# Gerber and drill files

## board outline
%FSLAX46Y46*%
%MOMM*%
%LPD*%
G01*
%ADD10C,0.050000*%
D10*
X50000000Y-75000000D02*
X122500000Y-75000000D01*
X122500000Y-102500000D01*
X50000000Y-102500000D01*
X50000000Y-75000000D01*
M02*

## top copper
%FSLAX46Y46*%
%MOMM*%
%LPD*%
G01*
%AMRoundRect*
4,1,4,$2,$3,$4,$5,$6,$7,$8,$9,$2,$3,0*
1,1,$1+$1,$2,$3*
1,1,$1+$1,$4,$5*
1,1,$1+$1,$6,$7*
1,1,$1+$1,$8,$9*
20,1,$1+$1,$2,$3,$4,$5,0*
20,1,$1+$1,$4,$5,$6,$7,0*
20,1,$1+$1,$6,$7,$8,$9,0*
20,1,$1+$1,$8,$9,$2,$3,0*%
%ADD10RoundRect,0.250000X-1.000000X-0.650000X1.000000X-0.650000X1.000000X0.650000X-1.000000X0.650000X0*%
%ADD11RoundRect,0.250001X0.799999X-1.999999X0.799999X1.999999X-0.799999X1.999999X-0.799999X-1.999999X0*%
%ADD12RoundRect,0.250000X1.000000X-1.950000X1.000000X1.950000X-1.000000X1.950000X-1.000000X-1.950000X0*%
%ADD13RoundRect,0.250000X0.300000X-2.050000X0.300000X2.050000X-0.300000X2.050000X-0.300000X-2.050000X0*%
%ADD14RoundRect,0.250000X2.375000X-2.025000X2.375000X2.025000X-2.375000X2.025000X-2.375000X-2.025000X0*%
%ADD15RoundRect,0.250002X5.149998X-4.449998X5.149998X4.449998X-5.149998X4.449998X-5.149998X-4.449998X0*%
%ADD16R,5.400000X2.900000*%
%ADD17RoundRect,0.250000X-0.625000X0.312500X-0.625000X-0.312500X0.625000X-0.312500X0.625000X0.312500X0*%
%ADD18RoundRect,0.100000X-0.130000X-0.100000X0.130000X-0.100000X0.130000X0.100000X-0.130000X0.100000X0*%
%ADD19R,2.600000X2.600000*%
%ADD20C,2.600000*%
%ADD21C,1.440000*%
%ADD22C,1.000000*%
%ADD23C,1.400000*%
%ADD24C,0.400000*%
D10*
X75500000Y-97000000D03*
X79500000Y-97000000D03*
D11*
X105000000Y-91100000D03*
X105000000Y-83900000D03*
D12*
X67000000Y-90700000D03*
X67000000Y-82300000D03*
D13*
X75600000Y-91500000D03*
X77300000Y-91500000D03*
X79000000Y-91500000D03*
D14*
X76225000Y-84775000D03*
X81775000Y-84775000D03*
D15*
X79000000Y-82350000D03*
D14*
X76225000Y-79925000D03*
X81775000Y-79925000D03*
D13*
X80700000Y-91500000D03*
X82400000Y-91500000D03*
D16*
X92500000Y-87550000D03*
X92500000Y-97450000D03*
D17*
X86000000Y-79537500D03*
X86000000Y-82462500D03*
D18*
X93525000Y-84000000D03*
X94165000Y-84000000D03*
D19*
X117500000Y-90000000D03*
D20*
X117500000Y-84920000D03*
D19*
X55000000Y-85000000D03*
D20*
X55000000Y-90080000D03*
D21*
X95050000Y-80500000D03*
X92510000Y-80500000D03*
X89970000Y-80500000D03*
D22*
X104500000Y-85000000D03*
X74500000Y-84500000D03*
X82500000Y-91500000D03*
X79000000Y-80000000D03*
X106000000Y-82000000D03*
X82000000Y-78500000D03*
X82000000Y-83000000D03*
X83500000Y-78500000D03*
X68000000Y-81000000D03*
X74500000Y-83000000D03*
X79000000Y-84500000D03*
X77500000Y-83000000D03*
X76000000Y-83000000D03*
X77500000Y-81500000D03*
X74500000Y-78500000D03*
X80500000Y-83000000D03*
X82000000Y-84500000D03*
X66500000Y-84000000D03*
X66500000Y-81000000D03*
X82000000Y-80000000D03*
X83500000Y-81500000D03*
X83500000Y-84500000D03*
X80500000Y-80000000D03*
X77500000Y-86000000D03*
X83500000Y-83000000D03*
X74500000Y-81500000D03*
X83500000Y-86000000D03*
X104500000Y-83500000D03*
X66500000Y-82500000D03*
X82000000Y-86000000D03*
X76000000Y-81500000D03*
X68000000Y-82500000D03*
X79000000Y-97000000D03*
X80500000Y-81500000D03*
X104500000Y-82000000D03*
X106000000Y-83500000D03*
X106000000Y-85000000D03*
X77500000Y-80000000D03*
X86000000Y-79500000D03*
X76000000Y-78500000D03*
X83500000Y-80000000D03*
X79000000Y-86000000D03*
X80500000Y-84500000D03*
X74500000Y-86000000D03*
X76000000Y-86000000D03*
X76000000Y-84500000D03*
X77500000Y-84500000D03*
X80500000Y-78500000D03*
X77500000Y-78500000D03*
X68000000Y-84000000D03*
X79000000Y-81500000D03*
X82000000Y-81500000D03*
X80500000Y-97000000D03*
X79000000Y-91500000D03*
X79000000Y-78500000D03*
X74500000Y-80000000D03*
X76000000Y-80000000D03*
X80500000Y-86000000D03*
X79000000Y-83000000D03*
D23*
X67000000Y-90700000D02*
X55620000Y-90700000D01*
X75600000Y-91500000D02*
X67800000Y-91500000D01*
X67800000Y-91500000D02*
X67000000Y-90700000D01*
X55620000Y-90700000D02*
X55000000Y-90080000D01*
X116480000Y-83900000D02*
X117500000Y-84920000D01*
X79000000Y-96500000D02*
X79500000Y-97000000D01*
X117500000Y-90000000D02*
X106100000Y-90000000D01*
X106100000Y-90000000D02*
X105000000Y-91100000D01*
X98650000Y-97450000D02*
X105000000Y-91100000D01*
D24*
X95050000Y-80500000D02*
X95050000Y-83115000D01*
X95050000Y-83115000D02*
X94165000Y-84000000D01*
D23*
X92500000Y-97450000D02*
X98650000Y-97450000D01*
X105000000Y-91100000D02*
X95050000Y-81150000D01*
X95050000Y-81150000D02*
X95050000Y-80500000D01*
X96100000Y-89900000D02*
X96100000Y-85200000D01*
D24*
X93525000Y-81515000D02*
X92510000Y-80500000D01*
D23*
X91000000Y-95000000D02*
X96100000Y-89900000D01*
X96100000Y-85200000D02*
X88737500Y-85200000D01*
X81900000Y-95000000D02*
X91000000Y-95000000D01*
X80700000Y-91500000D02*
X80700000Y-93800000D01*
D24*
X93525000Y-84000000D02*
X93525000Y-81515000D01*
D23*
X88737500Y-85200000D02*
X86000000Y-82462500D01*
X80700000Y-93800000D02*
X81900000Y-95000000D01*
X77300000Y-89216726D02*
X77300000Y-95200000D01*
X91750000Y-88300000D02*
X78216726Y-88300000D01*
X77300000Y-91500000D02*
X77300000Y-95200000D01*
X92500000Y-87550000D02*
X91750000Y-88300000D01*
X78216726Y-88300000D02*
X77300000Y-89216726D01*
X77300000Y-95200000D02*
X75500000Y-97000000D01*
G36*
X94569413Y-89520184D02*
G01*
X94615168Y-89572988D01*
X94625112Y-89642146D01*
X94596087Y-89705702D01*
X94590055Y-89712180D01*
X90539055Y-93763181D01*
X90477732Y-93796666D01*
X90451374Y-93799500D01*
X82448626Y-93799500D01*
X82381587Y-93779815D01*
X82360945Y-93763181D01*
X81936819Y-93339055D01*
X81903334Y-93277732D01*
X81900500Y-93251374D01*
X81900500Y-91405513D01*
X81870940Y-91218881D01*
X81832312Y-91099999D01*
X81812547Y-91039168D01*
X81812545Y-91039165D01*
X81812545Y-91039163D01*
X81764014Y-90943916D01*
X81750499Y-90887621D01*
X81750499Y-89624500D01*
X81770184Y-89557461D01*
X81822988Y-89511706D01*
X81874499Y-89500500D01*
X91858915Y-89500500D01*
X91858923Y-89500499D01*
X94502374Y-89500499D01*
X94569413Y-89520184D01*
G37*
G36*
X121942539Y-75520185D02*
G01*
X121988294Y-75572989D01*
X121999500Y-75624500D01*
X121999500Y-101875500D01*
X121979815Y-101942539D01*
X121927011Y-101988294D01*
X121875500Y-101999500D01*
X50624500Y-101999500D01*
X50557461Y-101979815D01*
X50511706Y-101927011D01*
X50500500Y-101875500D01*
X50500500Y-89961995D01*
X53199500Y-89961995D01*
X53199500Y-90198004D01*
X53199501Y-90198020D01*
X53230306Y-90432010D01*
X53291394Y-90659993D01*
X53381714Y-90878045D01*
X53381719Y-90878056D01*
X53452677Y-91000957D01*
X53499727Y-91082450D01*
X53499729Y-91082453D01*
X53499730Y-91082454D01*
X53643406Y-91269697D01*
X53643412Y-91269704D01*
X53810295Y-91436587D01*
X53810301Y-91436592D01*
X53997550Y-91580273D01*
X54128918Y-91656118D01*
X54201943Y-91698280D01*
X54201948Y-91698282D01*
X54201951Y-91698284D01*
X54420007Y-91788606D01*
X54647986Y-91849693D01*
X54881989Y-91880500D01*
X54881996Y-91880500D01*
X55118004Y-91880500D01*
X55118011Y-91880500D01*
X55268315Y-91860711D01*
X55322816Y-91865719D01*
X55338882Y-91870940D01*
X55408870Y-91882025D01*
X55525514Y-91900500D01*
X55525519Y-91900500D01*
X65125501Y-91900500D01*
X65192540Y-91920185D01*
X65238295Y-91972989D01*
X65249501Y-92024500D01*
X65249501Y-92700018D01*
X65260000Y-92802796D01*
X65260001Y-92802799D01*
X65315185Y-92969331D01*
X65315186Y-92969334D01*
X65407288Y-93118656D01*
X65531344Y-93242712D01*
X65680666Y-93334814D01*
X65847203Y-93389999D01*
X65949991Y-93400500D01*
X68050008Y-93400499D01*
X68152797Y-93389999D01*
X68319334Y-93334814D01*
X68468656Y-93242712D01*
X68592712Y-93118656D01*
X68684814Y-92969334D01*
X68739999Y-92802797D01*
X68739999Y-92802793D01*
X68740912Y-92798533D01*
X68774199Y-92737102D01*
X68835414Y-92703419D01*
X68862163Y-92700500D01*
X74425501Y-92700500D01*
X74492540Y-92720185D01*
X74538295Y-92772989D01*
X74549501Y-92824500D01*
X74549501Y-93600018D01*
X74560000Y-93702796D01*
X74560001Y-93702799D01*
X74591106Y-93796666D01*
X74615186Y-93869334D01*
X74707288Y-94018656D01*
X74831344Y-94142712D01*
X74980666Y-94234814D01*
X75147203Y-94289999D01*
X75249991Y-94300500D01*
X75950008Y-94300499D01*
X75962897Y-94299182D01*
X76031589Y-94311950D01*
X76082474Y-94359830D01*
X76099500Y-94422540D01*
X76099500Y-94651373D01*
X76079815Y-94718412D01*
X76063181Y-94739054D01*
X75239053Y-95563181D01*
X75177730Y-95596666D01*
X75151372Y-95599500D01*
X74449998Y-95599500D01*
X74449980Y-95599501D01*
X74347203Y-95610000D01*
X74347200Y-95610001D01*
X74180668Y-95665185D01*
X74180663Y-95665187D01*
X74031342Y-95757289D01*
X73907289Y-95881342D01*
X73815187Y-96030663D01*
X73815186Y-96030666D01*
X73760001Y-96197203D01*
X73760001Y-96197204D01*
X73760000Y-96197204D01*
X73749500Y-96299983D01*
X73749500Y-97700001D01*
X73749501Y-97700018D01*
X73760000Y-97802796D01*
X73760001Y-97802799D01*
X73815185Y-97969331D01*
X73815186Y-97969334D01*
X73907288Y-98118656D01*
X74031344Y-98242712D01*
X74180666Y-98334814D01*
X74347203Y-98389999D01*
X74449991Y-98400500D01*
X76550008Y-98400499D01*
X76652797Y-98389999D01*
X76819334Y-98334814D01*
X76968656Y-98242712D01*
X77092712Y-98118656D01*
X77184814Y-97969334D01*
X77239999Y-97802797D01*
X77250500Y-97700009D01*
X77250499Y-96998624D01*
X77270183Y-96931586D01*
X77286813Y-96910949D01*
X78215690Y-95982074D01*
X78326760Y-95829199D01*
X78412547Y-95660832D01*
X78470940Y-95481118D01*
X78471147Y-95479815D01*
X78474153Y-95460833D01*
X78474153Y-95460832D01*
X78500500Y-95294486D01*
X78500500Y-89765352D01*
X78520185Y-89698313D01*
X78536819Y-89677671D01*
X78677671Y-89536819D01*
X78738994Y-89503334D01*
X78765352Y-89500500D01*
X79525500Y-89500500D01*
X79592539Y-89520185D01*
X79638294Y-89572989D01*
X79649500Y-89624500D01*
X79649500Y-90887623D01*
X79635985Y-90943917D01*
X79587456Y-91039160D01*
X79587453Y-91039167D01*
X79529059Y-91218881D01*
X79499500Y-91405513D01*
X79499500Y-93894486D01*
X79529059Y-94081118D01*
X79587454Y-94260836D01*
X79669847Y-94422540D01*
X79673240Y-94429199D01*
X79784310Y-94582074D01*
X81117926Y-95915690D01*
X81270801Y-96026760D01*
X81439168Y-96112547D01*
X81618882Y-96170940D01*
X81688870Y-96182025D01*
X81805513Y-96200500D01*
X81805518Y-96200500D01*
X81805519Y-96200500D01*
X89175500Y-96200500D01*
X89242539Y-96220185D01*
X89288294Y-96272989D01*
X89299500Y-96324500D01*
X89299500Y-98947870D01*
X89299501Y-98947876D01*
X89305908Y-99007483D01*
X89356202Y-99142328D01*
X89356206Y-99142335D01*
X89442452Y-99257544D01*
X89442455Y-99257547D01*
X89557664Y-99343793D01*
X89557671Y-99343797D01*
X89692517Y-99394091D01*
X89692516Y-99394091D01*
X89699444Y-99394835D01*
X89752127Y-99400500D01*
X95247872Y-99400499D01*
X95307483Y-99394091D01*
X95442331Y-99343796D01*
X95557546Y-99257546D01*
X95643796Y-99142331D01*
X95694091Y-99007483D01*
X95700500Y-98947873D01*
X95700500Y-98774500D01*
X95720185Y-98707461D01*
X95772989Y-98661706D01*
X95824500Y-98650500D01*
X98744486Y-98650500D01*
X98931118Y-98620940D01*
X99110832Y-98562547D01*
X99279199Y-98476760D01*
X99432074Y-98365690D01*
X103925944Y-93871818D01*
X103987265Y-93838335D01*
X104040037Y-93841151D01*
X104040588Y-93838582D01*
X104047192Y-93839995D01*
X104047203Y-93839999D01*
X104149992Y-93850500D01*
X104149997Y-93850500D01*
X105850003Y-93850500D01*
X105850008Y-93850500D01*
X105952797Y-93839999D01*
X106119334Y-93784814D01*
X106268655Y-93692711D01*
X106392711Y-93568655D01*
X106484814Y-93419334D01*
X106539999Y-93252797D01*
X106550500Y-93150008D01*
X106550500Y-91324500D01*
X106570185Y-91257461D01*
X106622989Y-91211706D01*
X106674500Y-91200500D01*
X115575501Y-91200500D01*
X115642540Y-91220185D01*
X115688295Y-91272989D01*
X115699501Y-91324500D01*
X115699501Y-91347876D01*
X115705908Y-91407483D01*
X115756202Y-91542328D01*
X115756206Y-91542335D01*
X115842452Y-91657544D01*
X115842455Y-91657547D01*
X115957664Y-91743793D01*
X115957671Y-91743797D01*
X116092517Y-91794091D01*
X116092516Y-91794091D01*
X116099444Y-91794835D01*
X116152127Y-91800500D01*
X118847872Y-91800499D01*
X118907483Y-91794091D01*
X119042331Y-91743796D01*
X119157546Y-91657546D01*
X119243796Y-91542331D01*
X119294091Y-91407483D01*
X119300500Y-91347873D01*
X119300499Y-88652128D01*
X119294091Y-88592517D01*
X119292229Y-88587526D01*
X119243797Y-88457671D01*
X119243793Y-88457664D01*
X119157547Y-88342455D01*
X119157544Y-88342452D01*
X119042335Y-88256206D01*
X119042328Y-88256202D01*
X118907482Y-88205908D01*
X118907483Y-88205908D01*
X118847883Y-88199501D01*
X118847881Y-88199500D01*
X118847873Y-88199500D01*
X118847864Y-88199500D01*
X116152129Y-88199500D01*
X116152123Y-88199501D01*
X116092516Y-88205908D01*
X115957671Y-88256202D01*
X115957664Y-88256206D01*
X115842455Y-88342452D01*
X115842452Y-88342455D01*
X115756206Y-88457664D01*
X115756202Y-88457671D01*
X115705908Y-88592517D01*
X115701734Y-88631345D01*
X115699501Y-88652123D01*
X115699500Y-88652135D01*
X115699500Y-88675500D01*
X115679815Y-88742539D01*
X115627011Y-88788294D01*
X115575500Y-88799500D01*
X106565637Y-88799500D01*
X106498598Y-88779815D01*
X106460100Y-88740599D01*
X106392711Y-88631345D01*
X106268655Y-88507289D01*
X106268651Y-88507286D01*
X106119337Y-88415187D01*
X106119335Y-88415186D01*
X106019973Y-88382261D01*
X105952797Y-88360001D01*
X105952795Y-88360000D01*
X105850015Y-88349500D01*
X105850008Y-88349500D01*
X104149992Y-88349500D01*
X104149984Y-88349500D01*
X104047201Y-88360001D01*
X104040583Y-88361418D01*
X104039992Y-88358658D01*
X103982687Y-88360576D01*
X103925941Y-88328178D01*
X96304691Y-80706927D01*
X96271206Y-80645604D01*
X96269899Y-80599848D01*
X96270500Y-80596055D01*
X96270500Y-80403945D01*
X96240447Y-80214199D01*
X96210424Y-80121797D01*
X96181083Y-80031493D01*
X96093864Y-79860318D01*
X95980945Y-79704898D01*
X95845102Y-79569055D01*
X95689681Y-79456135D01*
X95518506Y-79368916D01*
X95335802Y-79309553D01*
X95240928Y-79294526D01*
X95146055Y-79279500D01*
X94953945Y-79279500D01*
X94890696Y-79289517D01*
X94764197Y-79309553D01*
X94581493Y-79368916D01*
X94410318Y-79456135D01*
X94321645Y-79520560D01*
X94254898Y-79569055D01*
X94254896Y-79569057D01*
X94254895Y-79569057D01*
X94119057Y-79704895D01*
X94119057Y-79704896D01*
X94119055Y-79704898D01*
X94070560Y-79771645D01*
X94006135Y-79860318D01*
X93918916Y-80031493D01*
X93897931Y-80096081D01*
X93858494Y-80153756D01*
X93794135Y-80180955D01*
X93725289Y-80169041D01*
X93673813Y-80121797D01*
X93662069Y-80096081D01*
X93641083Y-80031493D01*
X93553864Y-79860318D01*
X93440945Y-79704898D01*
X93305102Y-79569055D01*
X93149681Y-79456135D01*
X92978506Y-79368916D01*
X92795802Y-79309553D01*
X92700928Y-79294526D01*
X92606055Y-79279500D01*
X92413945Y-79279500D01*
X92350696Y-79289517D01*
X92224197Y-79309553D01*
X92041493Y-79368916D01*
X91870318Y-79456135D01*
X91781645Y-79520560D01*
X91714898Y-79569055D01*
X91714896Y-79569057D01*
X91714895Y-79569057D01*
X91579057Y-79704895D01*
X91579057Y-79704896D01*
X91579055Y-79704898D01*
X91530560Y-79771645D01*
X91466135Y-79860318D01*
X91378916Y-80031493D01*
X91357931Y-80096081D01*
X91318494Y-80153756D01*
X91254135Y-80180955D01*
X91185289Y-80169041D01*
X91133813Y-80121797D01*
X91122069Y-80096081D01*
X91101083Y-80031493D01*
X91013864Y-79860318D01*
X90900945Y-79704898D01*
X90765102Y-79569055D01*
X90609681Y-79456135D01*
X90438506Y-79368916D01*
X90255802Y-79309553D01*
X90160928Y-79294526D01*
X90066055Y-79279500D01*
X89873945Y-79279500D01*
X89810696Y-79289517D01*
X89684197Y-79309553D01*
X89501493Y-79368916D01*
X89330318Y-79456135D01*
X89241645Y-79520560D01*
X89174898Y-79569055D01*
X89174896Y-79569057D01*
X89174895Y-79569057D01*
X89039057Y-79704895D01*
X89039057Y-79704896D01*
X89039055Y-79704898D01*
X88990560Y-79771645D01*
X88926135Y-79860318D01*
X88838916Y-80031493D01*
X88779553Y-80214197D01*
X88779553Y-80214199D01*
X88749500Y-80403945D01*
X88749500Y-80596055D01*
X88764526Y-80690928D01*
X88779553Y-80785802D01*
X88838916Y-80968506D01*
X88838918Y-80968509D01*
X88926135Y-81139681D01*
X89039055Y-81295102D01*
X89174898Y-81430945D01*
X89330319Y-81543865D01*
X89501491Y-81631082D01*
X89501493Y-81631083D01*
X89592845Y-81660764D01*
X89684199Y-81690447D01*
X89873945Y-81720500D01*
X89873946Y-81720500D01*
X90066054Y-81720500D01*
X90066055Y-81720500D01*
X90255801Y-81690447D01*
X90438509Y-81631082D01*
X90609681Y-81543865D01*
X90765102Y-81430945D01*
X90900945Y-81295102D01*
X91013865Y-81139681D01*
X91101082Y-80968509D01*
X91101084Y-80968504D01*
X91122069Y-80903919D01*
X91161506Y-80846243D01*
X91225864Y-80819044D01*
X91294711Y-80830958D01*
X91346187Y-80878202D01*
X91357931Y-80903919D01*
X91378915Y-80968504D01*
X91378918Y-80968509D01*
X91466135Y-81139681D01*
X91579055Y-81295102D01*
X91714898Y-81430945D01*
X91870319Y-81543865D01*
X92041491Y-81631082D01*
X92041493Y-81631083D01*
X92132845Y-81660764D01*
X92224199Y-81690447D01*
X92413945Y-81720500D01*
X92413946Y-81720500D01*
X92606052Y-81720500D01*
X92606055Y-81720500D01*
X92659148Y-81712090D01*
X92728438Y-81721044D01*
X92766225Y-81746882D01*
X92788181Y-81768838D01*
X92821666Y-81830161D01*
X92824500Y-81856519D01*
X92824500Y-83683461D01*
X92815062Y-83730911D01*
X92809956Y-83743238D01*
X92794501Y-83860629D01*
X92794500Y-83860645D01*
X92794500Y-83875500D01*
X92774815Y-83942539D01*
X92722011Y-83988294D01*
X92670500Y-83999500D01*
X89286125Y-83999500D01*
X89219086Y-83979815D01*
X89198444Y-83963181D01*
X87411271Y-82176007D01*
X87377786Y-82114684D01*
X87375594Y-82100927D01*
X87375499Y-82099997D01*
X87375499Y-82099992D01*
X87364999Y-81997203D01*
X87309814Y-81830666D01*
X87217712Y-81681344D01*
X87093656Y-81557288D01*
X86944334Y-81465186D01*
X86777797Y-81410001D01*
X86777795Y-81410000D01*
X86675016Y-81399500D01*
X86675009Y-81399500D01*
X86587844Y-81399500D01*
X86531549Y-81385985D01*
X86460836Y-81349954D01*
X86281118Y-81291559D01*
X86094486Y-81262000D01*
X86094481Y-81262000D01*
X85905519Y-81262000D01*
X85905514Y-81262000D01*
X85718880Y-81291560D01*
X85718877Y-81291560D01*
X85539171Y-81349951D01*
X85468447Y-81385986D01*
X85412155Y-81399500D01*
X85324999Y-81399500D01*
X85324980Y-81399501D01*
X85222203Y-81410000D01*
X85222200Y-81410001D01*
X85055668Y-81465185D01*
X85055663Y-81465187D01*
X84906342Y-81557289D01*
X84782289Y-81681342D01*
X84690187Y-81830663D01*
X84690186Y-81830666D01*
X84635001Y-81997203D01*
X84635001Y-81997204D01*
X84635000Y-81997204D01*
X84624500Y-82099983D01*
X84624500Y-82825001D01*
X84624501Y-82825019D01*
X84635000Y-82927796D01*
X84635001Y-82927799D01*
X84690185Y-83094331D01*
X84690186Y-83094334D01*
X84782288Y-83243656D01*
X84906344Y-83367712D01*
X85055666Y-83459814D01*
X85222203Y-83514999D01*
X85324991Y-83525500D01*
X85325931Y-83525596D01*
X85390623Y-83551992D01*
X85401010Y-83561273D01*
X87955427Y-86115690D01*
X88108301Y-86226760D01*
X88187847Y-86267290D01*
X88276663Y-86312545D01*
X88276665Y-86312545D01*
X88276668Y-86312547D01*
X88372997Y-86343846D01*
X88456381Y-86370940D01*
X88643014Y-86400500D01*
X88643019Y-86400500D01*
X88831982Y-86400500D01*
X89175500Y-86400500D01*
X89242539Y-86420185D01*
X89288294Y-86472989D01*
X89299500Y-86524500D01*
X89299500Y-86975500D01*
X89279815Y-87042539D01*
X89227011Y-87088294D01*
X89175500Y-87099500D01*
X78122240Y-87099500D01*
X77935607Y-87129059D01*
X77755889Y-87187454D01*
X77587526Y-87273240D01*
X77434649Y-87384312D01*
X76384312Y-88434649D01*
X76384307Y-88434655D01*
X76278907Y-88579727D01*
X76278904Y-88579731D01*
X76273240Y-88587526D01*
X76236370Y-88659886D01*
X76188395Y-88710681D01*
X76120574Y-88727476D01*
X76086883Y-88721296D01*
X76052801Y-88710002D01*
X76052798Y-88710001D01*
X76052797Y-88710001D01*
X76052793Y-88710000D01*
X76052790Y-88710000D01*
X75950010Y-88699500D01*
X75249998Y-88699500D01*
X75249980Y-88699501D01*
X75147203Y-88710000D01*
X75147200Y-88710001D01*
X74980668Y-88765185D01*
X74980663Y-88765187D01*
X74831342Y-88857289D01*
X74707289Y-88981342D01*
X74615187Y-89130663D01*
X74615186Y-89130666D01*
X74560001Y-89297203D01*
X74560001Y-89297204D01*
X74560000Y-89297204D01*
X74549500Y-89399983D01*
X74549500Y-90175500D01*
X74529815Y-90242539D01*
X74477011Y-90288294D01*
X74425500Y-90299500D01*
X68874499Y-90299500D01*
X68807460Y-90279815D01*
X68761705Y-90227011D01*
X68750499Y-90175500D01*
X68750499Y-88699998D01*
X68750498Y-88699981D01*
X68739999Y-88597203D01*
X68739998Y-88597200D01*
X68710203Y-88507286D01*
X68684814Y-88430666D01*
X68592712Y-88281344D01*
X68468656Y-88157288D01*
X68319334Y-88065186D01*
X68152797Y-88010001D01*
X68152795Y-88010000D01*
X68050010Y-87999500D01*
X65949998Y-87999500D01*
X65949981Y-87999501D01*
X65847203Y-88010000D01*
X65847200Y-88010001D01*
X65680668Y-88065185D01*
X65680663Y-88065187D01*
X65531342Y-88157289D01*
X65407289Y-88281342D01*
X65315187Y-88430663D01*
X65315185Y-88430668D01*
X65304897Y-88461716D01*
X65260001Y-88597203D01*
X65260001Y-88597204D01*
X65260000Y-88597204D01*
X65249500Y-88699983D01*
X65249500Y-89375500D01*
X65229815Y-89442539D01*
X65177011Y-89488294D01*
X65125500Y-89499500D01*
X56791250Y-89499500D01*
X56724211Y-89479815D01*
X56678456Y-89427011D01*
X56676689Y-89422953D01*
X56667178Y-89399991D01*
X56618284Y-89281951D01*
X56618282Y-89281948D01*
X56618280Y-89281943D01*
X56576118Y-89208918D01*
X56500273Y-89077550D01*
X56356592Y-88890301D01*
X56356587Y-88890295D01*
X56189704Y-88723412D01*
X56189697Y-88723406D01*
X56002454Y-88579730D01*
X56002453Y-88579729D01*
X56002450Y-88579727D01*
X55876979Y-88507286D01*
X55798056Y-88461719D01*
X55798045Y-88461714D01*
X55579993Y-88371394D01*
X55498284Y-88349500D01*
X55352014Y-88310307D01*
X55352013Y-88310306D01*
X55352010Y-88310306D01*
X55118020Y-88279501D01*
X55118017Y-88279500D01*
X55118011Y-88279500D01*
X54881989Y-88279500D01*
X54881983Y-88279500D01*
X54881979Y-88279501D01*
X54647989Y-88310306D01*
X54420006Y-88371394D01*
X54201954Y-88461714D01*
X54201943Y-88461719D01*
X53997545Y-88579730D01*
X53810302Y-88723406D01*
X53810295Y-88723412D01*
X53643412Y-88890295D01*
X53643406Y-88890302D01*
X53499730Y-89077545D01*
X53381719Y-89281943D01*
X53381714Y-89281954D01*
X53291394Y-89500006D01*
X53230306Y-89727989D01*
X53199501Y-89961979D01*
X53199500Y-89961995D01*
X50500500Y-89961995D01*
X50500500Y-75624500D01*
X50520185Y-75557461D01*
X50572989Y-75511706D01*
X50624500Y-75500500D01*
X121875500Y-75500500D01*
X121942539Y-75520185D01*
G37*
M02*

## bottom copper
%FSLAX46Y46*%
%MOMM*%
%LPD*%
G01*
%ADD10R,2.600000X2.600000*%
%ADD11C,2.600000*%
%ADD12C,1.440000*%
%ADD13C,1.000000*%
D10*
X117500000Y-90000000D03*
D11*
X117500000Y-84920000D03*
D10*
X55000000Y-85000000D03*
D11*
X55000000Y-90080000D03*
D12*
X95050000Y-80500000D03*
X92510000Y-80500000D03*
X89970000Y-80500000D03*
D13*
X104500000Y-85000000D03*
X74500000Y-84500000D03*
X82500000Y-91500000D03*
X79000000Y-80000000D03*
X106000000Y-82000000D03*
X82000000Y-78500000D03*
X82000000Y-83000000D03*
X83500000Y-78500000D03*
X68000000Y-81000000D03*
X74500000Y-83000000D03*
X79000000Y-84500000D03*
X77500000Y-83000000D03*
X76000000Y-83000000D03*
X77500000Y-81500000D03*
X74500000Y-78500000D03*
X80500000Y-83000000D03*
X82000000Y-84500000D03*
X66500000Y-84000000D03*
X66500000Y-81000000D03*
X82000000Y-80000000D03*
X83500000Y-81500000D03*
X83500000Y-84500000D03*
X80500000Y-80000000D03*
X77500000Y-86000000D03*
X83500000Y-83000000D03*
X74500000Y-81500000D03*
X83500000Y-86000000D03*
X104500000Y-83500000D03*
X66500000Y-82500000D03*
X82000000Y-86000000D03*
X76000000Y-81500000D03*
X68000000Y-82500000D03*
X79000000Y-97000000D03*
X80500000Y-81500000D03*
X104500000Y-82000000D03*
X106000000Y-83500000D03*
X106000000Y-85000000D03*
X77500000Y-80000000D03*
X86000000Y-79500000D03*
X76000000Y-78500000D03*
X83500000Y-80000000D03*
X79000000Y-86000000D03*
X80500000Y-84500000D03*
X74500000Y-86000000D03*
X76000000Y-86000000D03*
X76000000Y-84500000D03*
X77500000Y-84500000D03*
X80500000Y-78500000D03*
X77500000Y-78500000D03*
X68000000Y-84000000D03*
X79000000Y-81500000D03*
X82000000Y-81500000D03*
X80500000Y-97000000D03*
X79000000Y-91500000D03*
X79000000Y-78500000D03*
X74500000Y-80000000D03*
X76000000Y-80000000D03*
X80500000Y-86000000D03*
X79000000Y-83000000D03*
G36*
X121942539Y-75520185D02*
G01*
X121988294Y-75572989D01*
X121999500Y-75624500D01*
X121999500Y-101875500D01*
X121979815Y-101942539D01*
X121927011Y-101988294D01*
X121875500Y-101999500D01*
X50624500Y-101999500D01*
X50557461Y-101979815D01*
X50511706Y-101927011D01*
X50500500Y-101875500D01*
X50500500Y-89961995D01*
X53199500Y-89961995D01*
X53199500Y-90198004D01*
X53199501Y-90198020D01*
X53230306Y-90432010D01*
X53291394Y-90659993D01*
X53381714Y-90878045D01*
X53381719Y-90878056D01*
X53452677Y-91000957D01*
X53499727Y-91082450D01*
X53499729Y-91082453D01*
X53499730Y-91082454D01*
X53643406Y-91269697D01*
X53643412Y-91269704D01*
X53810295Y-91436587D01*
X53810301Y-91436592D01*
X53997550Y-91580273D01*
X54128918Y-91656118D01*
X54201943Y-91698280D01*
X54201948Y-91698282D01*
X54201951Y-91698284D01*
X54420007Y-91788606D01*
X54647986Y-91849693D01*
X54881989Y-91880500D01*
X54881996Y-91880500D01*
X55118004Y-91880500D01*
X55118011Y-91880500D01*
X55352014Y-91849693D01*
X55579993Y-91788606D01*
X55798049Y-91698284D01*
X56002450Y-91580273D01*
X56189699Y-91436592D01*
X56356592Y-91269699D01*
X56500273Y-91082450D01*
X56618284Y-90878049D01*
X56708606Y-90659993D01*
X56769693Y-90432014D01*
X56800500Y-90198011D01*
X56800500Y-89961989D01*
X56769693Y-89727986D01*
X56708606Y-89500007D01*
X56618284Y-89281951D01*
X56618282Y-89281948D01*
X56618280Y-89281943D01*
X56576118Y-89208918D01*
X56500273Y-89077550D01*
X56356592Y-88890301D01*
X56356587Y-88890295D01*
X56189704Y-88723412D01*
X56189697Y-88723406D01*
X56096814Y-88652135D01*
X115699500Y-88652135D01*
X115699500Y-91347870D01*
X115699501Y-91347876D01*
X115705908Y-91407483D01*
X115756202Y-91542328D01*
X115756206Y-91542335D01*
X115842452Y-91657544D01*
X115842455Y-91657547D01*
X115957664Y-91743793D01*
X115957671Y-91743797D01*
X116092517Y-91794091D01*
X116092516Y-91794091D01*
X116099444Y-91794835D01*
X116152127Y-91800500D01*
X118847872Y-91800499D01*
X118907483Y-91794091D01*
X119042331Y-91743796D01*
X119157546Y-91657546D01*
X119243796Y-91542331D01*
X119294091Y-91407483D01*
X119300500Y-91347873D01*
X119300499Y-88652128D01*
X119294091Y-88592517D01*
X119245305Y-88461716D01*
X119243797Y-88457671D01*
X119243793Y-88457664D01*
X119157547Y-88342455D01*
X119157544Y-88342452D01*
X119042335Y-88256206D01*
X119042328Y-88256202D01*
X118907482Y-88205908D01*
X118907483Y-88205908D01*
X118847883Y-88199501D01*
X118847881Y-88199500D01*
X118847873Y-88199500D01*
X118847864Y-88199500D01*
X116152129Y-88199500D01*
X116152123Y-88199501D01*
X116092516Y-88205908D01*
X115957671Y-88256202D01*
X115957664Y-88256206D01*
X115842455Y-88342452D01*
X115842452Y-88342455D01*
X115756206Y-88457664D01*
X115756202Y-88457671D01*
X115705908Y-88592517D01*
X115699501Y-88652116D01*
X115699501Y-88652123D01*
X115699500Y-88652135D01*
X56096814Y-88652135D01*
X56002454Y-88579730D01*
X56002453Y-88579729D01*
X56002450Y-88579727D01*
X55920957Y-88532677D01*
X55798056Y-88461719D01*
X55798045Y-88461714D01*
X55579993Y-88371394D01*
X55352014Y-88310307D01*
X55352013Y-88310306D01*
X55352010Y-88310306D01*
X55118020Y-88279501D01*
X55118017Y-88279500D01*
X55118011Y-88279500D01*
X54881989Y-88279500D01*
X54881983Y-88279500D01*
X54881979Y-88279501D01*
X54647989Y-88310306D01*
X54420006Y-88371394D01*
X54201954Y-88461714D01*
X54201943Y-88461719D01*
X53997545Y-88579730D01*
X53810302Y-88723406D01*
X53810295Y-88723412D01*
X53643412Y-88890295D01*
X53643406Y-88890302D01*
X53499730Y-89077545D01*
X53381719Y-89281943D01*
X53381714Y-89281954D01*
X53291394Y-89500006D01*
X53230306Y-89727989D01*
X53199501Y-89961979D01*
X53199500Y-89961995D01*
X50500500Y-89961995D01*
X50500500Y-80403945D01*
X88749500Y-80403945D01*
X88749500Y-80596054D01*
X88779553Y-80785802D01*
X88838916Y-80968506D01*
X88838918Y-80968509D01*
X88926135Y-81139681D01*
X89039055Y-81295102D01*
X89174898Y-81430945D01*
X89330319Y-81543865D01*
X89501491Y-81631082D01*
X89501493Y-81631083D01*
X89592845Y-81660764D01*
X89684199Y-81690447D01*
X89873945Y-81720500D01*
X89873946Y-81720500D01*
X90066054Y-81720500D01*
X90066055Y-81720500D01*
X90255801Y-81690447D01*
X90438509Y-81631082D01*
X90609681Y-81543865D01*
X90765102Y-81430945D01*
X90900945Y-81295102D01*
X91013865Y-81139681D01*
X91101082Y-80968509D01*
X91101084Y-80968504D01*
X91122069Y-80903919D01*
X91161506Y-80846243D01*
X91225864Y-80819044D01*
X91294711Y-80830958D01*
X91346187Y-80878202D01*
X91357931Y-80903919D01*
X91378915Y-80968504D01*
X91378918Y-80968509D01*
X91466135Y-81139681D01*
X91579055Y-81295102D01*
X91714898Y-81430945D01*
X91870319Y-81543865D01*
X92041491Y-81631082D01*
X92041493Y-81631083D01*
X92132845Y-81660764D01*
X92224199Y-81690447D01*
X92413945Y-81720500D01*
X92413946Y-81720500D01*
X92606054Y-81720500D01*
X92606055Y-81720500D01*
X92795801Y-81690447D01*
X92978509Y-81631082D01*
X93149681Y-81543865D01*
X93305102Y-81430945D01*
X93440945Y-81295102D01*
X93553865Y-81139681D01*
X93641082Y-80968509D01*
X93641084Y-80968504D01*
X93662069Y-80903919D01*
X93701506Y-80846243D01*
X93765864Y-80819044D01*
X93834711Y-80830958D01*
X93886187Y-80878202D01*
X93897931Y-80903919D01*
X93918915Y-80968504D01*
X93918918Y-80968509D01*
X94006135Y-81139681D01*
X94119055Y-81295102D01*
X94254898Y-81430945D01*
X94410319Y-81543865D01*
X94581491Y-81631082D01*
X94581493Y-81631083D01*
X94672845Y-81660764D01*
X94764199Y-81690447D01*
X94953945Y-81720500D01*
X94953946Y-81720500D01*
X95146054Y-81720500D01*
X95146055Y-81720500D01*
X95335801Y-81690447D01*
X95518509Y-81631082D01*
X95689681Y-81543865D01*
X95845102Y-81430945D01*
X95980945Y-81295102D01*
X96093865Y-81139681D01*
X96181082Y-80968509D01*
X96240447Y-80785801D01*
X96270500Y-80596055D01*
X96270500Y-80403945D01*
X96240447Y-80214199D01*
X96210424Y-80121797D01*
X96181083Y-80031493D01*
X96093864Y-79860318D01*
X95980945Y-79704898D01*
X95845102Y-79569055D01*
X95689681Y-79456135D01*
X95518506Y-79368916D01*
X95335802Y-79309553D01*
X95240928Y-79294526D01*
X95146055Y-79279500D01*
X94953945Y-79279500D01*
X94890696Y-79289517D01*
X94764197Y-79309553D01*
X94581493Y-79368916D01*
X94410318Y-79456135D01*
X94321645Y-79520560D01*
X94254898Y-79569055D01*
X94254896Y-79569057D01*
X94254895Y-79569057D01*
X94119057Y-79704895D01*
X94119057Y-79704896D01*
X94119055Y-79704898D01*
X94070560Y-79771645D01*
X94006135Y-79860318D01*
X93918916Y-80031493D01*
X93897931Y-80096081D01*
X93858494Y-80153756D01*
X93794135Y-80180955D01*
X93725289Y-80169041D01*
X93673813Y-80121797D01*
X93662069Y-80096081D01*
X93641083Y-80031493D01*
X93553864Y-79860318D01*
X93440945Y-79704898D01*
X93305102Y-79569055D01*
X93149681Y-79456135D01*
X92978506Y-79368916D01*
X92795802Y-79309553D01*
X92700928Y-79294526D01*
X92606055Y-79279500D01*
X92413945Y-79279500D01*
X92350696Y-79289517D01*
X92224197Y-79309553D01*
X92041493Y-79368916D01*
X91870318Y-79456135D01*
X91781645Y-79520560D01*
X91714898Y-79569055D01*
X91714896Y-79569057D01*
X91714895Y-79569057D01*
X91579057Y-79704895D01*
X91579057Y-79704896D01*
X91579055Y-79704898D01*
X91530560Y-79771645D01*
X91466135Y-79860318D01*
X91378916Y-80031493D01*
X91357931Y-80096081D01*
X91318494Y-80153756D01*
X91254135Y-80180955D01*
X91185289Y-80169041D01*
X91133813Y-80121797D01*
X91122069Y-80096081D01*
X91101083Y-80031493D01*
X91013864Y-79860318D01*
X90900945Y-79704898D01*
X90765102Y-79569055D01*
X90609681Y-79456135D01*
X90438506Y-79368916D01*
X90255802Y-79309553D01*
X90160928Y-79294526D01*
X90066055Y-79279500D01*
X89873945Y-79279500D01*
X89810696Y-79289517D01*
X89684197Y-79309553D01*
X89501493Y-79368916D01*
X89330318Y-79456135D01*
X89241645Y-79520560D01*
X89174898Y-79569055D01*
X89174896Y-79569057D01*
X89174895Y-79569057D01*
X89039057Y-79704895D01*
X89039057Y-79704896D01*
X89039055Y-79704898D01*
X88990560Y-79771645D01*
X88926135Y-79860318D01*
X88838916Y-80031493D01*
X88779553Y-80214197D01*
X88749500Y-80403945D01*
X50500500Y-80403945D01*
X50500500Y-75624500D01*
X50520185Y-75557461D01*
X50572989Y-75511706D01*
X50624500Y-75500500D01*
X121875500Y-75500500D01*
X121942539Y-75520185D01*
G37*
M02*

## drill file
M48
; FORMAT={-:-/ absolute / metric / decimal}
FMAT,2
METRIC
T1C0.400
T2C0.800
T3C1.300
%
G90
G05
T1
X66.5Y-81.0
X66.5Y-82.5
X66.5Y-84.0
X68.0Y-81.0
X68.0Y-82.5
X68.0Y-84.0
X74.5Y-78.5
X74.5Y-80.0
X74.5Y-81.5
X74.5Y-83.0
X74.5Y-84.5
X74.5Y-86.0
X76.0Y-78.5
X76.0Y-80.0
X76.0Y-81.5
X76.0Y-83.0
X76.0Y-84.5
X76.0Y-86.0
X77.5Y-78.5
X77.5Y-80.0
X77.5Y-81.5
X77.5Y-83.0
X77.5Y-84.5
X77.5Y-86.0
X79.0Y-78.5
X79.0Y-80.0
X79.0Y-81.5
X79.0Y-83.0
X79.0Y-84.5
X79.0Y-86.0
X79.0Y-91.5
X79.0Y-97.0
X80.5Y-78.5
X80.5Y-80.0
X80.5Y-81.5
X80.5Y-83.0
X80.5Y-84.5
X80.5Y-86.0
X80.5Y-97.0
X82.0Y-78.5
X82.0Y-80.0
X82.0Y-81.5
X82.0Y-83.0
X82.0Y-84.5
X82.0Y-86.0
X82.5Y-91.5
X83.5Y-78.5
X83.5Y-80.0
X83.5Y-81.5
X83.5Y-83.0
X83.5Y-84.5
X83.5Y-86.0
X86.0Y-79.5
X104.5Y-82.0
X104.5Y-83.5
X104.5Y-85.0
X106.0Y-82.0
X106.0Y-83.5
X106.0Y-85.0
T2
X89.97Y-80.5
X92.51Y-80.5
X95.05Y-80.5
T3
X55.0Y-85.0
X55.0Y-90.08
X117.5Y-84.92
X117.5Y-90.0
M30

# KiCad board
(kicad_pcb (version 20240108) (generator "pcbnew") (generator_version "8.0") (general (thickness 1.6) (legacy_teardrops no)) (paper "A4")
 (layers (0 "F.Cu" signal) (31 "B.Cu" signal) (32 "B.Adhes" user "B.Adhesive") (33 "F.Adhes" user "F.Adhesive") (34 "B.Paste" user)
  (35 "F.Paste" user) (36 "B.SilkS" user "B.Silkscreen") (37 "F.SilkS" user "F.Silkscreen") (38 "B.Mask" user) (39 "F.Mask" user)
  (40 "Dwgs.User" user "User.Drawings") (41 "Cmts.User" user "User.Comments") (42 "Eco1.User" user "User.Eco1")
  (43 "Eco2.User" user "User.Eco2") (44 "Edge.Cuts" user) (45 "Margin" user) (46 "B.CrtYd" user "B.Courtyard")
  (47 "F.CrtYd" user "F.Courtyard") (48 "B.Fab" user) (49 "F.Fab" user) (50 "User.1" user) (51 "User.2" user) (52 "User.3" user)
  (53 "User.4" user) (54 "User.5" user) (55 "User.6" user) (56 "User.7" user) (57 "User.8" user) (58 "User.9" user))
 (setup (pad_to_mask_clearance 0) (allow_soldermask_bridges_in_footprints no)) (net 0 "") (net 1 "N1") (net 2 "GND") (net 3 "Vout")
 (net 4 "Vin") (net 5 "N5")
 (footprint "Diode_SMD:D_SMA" (layer "F.Cu") (at 77.5 97)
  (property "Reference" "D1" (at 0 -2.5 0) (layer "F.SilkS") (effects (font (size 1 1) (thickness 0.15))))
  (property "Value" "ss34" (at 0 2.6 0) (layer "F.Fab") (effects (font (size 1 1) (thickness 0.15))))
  (pad "1" smd roundrect (at -2 0) (size 2.5 1.8) (layers "F.Cu" "F.Paste" "F.Mask") (roundrect_rratio 0.1388888889) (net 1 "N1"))
  (pad "2" smd roundrect (at 2 0) (size 2.5 1.8) (layers "F.Cu" "F.Paste" "F.Mask") (roundrect_rratio 0.1388888889) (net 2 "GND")))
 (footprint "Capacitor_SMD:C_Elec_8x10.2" (layer "F.Cu") (at 105 87.5 90)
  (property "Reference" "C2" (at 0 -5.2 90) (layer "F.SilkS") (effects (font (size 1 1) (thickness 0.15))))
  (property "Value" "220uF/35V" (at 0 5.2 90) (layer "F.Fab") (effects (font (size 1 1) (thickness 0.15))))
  (pad "1" smd roundrect (at -3.6 0 90) (size 4.5 2.1) (layers "F.Cu" "F.Paste" "F.Mask") (roundrect_rratio 0.119048) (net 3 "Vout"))
  (pad "2" smd roundrect (at 3.6 0 90) (size 4.5 2.1) (layers "F.Cu" "F.Paste" "F.Mask") (roundrect_rratio 0.119048) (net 2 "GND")))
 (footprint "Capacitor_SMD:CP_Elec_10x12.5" (layer "F.Cu") (at 67 86.5 90)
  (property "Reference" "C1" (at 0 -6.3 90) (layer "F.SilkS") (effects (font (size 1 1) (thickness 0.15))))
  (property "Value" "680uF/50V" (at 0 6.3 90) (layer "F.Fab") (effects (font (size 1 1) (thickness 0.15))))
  (pad "1" smd roundrect (at -4.2 0 90) (size 4.4 2.5) (layers "F.Cu" "F.Paste" "F.Mask") (roundrect_rratio 0.1) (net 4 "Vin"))
  (pad "2" smd roundrect (at 4.2 0 90) (size 4.4 2.5) (layers "F.Cu" "F.Paste" "F.Mask") (roundrect_rratio 0.1) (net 2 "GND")))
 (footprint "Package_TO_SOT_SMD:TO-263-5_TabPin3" (layer "F.Cu") (at 79 83.85 90)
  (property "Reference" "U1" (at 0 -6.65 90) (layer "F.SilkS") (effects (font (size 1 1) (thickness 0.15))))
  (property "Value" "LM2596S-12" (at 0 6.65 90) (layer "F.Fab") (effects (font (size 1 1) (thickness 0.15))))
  (pad "1" smd roundrect (at -7.65 -3.4 90) (size 4.6 1.1) (layers "F.Cu" "F.Paste" "F.Mask") (roundrect_rratio 0.227273) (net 4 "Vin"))
  (pad "2" smd roundrect (at -7.65 -1.7 90) (size 4.6 1.1) (layers "F.Cu" "F.Paste" "F.Mask") (roundrect_rratio 0.227273) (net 1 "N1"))
  (pad "3" smd roundrect (at -7.65 0 90) (size 4.6 1.1) (layers "F.Cu" "F.Paste" "F.Mask") (roundrect_rratio 0.227273) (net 2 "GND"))
  (pad "3" smd roundrect (at -0.925 -2.775 90) (size 4.55 5.25) (layers "F.Cu" "F.Paste") (roundrect_rratio 0.054945) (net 2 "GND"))
  (pad "3" smd roundrect (at -0.925 2.775 90) (size 4.55 5.25) (layers "F.Cu" "F.Paste") (roundrect_rratio 0.054945) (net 2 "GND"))
  (pad "3" smd roundrect (at 1.5 0 90) (size 9.4 10.8) (layers "F.Cu" "F.Mask") (roundrect_rratio 0.026596) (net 2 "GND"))
  (pad "3" smd roundrect (at 3.925 -2.775 90) (size 4.55 5.25) (layers "F.Cu" "F.Paste") (roundrect_rratio 0.054945) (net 2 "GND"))
  (pad "3" smd roundrect (at 3.925 2.775 90) (size 4.55 5.25) (layers "F.Cu" "F.Paste") (roundrect_rratio 0.054945) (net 2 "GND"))
  (pad "4" smd roundrect (at -7.65 1.7 90) (size 4.6 1.1) (layers "F.Cu" "F.Paste" "F.Mask") (roundrect_rratio 0.227273) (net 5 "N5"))
  (pad "5" smd roundrect (at -7.65 3.4 90) (size 4.6 1.1) (layers "F.Cu" "F.Paste" "F.Mask") (roundrect_rratio 0.227273) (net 2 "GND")))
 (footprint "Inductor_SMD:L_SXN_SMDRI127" (layer "F.Cu") (at 92.5 92.5 -90)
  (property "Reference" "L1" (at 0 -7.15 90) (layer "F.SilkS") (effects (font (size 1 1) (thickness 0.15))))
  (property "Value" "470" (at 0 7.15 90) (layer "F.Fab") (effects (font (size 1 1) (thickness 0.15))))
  (pad "1" smd rect (at -4.95 0 270) (size 2.9 5.4) (layers "F.Cu" "F.Paste" "F.Mask") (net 1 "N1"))
  (pad "2" smd rect (at 4.95 0 270) (size 2.9 5.4) (layers "F.Cu" "F.Paste" "F.Mask") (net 3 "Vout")))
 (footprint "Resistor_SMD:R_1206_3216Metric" (layer "F.Cu") (at 86 81 -90)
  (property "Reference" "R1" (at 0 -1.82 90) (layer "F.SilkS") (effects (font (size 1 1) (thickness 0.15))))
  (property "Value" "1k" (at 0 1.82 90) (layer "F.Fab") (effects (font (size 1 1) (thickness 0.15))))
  (pad "1" smd roundrect (at -1.4625 0 270) (size 1.125 1.75) (layers "F.Cu" "F.Paste" "F.Mask") (roundrect_rratio 0.222222) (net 2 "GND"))
  (pad "2" smd roundrect (at 1.4625 0 270) (size 1.125 1.75) (layers "F.Cu" "F.Paste" "F.Mask") (roundrect_rratio 0.222222) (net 5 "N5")))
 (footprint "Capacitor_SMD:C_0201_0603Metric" (layer "F.Cu") (at 93.845 84)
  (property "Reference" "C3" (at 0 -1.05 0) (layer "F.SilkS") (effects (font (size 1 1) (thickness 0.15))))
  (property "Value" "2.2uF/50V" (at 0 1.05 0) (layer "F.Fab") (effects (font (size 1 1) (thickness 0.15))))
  (pad "" smd roundrect (at -0.345 0) (size 0.318 0.36) (layers "F.Paste") (roundrect_rratio 0.25))
  (pad "" smd roundrect (at 0.345 0) (size 0.318 0.36) (layers "F.Paste") (roundrect_rratio 0.25))
  (pad "1" smd roundrect (at -0.32 0) (size 0.46 0.4) (layers "F.Cu" "F.Mask") (roundrect_rratio 0.25) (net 5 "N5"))
  (pad "2" smd roundrect (at 0.32 0) (size 0.46 0.4) (layers "F.Cu" "F.Mask") (roundrect_rratio 0.25) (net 3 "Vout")))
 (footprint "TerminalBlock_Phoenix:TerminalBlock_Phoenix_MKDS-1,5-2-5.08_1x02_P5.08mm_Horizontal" (layer "F.Cu") (at 117.5 90 90)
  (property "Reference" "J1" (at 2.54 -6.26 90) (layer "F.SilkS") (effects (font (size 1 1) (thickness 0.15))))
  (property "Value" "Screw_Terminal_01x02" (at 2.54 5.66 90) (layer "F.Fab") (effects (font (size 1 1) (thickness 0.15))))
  (pad "1" thru_hole rect (at 0 0 90) (size 2.6 2.6) (drill 1.3) (layers "*.Cu" "*.Mask") (remove_unused_layers no) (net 3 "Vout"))
  (pad "2" thru_hole circle (at 5.08 0 90) (size 2.6 2.6) (drill 1.3) (layers "*.Cu" "*.Mask") (remove_unused_layers no) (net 2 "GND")))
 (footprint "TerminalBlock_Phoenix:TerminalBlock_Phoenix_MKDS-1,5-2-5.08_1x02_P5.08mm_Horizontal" (layer "F.Cu") (at 55 85 -90)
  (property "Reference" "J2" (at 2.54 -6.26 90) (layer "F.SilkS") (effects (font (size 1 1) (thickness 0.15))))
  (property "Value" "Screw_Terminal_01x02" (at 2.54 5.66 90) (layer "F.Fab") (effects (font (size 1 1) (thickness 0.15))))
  (pad "1" thru_hole rect (at 0 0 270) (size 2.6 2.6) (drill 1.3) (layers "*.Cu" "*.Mask") (remove_unused_layers no) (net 2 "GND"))
  (pad "2" thru_hole circle (at 5.08 0 270) (size 2.6 2.6) (drill 1.3) (layers "*.Cu" "*.Mask") (remove_unused_layers no) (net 4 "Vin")))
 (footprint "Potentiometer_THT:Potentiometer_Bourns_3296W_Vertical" (layer "F.Cu") (at 95.05 80.5)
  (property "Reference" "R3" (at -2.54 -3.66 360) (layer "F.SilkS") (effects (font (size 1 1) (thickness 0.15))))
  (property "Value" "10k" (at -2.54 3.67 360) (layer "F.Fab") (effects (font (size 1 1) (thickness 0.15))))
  (pad "1" thru_hole circle (at 0 0) (size 1.44 1.44) (drill 0.8) (layers "*.Cu" "*.Mask") (remove_unused_layers no) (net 3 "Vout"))
  (pad "2" thru_hole circle (at -2.54 0) (size 1.44 1.44) (drill 0.8) (layers "*.Cu" "*.Mask") (remove_unused_layers no) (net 5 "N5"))
  (pad "3" thru_hole circle (at -5.08 0) (size 1.44 1.44) (drill 0.8) (layers "*.Cu" "*.Mask") (remove_unused_layers no)))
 (gr_rect (start 50 75) (end 122.5 102.5) (stroke (width 0.05) (type default)) (fill none) (layer "Edge.Cuts"))
 (segment (start 67 90.7) (end 55.62 90.7) (width 1.4) (layer "F.Cu") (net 4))
 (segment (start 75.6 91.5) (end 67.8 91.5) (width 1.4) (layer "F.Cu") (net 4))
 (segment (start 67.8 91.5) (end 67 90.7) (width 1.4) (layer "F.Cu") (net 4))
 (segment (start 55.62 90.7) (end 55 90.08) (width 1.4) (layer "F.Cu") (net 4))
 (segment (start 116.48 83.9) (end 117.5 84.92) (width 1.4) (layer "F.Cu") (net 2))
 (segment (start 79 96.5) (end 79.5 97) (width 1.4) (layer "F.Cu") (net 2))
 (via (at 104.5 85) (size 1) (drill 0.4) (layers "F.Cu" "B.Cu") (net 2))
 (via (at 74.5 84.5) (size 1) (drill 0.4) (layers "F.Cu" "B.Cu") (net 2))
 (via (at 82.5 91.5) (size 1) (drill 0.4) (layers "F.Cu" "B.Cu") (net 2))
 (via (at 79 80) (size 1) (drill 0.4) (layers "F.Cu" "B.Cu") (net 2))
 (via (at 106 82) (size 1) (drill 0.4) (layers "F.Cu" "B.Cu") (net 2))
 (via (at 82 78.5) (size 1) (drill 0.4) (layers "F.Cu" "B.Cu") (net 2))
 (via (at 82 83) (size 1) (drill 0.4) (layers "F.Cu" "B.Cu") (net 2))
 (via (at 83.5 78.5) (size 1) (drill 0.4) (layers "F.Cu" "B.Cu") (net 2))
 (via (at 68 81) (size 1) (drill 0.4) (layers "F.Cu" "B.Cu") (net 2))
 (via (at 74.5 83) (size 1) (drill 0.4) (layers "F.Cu" "B.Cu") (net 2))
 (via (at 79 84.5) (size 1) (drill 0.4) (layers "F.Cu" "B.Cu") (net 2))
 (via (at 77.5 83) (size 1) (drill 0.4) (layers "F.Cu" "B.Cu") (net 2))
 (via (at 76 83) (size 1) (drill 0.4) (layers "F.Cu" "B.Cu") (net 2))
 (via (at 77.5 81.5) (size 1) (drill 0.4) (layers "F.Cu" "B.Cu") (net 2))
 (via (at 74.5 78.5) (size 1) (drill 0.4) (layers "F.Cu" "B.Cu") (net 2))
 (via (at 80.5 83) (size 1) (drill 0.4) (layers "F.Cu" "B.Cu") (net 2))
 (via (at 82 84.5) (size 1) (drill 0.4) (layers "F.Cu" "B.Cu") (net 2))
 (via (at 66.5 84) (size 1) (drill 0.4) (layers "F.Cu" "B.Cu") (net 2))
 (via (at 66.5 81) (size 1) (drill 0.4) (layers "F.Cu" "B.Cu") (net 2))
 (via (at 82 80) (size 1) (drill 0.4) (layers "F.Cu" "B.Cu") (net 2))
 (via (at 83.5 81.5) (size 1) (drill 0.4) (layers "F.Cu" "B.Cu") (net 2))
 (via (at 83.5 84.5) (size 1) (drill 0.4) (layers "F.Cu" "B.Cu") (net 2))
 (via (at 80.5 80) (size 1) (drill 0.4) (layers "F.Cu" "B.Cu") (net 2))
 (via (at 77.5 86) (size 1) (drill 0.4) (layers "F.Cu" "B.Cu") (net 2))
 (via (at 83.5 83) (size 1) (drill 0.4) (layers "F.Cu" "B.Cu") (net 2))
 (via (at 74.5 81.5) (size 1) (drill 0.4) (layers "F.Cu" "B.Cu") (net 2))
 (via (at 83.5 86) (size 1) (drill 0.4) (layers "F.Cu" "B.Cu") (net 2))
 (via (at 104.5 83.5) (size 1) (drill 0.4) (layers "F.Cu" "B.Cu") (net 2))
 (via (at 66.5 82.5) (size 1) (drill 0.4) (layers "F.Cu" "B.Cu") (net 2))
 (via (at 82 86) (size 1) (drill 0.4) (layers "F.Cu" "B.Cu") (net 2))
 (via (at 76 81.5) (size 1) (drill 0.4) (layers "F.Cu" "B.Cu") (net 2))
 (via (at 68 82.5) (size 1) (drill 0.4) (layers "F.Cu" "B.Cu") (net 2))
 (via (at 79 97) (size 1) (drill 0.4) (layers "F.Cu" "B.Cu") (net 2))
 (via (at 80.5 81.5) (size 1) (drill 0.4) (layers "F.Cu" "B.Cu") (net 2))
 (via (at 104.5 82) (size 1) (drill 0.4) (layers "F.Cu" "B.Cu") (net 2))
 (via (at 106 83.5) (size 1) (drill 0.4) (layers "F.Cu" "B.Cu") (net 2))
 (via (at 106 85) (size 1) (drill 0.4) (layers "F.Cu" "B.Cu") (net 2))
 (via (at 77.5 80) (size 1) (drill 0.4) (layers "F.Cu" "B.Cu") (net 2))
 (via (at 86 79.5) (size 1) (drill 0.4) (layers "F.Cu" "B.Cu") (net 2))
 (via (at 76 78.5) (size 1) (drill 0.4) (layers "F.Cu" "B.Cu") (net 2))
 (via (at 83.5 80) (size 1) (drill 0.4) (layers "F.Cu" "B.Cu") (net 2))
 (via (at 79 86) (size 1) (drill 0.4) (layers "F.Cu" "B.Cu") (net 2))
 (via (at 80.5 84.5) (size 1) (drill 0.4) (layers "F.Cu" "B.Cu") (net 2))
 (via (at 74.5 86) (size 1) (drill 0.4) (layers "F.Cu" "B.Cu") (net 2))
 (via (at 76 86) (size 1) (drill 0.4) (layers "F.Cu" "B.Cu") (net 2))
 (via (at 76 84.5) (size 1) (drill 0.4) (layers "F.Cu" "B.Cu") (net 2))
 (via (at 77.5 84.5) (size 1) (drill 0.4) (layers "F.Cu" "B.Cu") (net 2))
 (via (at 80.5 78.5) (size 1) (drill 0.4) (layers "F.Cu" "B.Cu") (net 2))
 (via (at 77.5 78.5) (size 1) (drill 0.4) (layers "F.Cu" "B.Cu") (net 2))
 (via (at 68 84) (size 1) (drill 0.4) (layers "F.Cu" "B.Cu") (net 2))
 (via (at 79 81.5) (size 1) (drill 0.4) (layers "F.Cu" "B.Cu") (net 2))
 (via (at 82 81.5) (size 1) (drill 0.4) (layers "F.Cu" "B.Cu") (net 2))
 (via (at 80.5 97) (size 1) (drill 0.4) (layers "F.Cu" "B.Cu") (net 2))
 (via (at 79 91.5) (size 1) (drill 0.4) (layers "F.Cu" "B.Cu") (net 2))
 (via (at 79 78.5) (size 1) (drill 0.4) (layers "F.Cu" "B.Cu") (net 2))
 (via (at 74.5 80) (size 1) (drill 0.4) (layers "F.Cu" "B.Cu") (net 2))
 (via (at 76 80) (size 1) (drill 0.4) (layers "F.Cu" "B.Cu") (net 2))
 (via (at 80.5 86) (size 1) (drill 0.4) (layers "F.Cu" "B.Cu") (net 2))
 (via (at 79 83) (size 1) (drill 0.4) (layers "F.Cu" "B.Cu") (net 2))
 (segment (start 117.5 90) (end 106.1 90) (width 1.4) (layer "F.Cu") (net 3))
 (segment (start 106.1 90) (end 105 91.1) (width 1.4) (layer "F.Cu") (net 3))
 (segment (start 98.65 97.45) (end 105 91.1) (width 1.4) (layer "F.Cu") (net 3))
 (segment (start 95.05 80.5) (end 95.05 83.115) (width 0.4) (layer "F.Cu") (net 3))
 (segment (start 95.05 83.115) (end 94.165 84) (width 0.4) (layer "F.Cu") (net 3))
 (segment (start 92.5 97.45) (end 98.65 97.45) (width 1.4) (layer "F.Cu") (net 3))
 (segment (start 105 91.1) (end 95.05 81.15) (width 1.4) (layer "F.Cu") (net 3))
 (segment (start 95.05 81.15) (end 95.05 80.5) (width 1.4) (layer "F.Cu") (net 3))
 (segment (start 96.1 89.9) (end 96.1 85.2) (width 1.4) (layer "F.Cu") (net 5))
 (segment (start 93.525 81.515) (end 92.51 80.5) (width 0.4) (layer "F.Cu") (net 5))
 (segment (start 91 95) (end 96.1 89.9) (width 1.4) (layer "F.Cu") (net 5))
 (segment (start 96.1 85.2) (end 88.7375 85.2) (width 1.4) (layer "F.Cu") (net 5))
 (segment (start 81.9 95) (end 91 95) (width 1.4) (layer "F.Cu") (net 5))
 (segment (start 80.7 91.5) (end 80.7 93.8) (width 1.4) (layer "F.Cu") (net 5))
 (segment (start 93.525 84) (end 93.525 81.515) (width 0.4) (layer "F.Cu") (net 5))
 (segment (start 88.7375 85.2) (end 86 82.4625) (width 1.4) (layer "F.Cu") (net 5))
 (segment (start 80.7 93.8) (end 81.9 95) (width 1.4) (layer "F.Cu") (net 5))
 (segment (start 77.3 89.216726) (end 77.3 95.2) (width 1.4) (layer "F.Cu") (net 1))
 (segment (start 91.75 88.3) (end 78.216726 88.3) (width 1.4) (layer "F.Cu") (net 1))
 (segment (start 77.3 91.5) (end 77.3 95.2) (width 1.4) (layer "F.Cu") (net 1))
 (segment (start 92.5 87.55) (end 91.75 88.3) (width 1.4) (layer "F.Cu") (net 1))
 (segment (start 78.216726 88.3) (end 77.3 89.216726) (width 1.4) (layer "F.Cu") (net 1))
 (segment (start 77.3 95.2) (end 75.5 97) (width 1.4) (layer "F.Cu") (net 1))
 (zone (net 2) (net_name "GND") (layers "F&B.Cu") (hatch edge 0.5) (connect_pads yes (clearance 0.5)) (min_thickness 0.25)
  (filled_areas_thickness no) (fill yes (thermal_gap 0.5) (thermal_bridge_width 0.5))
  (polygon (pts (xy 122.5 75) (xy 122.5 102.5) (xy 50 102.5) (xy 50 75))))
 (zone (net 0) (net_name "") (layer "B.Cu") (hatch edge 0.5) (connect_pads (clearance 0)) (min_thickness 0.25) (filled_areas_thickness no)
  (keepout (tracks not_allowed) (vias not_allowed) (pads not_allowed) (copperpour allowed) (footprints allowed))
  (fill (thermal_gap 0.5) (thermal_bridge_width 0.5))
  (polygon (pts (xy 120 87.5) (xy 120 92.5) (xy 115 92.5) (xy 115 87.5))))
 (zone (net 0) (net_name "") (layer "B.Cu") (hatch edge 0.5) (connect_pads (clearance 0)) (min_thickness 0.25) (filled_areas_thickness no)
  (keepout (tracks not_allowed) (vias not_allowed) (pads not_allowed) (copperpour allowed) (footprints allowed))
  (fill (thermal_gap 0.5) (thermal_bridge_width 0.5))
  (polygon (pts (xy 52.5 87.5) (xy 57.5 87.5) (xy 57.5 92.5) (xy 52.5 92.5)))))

